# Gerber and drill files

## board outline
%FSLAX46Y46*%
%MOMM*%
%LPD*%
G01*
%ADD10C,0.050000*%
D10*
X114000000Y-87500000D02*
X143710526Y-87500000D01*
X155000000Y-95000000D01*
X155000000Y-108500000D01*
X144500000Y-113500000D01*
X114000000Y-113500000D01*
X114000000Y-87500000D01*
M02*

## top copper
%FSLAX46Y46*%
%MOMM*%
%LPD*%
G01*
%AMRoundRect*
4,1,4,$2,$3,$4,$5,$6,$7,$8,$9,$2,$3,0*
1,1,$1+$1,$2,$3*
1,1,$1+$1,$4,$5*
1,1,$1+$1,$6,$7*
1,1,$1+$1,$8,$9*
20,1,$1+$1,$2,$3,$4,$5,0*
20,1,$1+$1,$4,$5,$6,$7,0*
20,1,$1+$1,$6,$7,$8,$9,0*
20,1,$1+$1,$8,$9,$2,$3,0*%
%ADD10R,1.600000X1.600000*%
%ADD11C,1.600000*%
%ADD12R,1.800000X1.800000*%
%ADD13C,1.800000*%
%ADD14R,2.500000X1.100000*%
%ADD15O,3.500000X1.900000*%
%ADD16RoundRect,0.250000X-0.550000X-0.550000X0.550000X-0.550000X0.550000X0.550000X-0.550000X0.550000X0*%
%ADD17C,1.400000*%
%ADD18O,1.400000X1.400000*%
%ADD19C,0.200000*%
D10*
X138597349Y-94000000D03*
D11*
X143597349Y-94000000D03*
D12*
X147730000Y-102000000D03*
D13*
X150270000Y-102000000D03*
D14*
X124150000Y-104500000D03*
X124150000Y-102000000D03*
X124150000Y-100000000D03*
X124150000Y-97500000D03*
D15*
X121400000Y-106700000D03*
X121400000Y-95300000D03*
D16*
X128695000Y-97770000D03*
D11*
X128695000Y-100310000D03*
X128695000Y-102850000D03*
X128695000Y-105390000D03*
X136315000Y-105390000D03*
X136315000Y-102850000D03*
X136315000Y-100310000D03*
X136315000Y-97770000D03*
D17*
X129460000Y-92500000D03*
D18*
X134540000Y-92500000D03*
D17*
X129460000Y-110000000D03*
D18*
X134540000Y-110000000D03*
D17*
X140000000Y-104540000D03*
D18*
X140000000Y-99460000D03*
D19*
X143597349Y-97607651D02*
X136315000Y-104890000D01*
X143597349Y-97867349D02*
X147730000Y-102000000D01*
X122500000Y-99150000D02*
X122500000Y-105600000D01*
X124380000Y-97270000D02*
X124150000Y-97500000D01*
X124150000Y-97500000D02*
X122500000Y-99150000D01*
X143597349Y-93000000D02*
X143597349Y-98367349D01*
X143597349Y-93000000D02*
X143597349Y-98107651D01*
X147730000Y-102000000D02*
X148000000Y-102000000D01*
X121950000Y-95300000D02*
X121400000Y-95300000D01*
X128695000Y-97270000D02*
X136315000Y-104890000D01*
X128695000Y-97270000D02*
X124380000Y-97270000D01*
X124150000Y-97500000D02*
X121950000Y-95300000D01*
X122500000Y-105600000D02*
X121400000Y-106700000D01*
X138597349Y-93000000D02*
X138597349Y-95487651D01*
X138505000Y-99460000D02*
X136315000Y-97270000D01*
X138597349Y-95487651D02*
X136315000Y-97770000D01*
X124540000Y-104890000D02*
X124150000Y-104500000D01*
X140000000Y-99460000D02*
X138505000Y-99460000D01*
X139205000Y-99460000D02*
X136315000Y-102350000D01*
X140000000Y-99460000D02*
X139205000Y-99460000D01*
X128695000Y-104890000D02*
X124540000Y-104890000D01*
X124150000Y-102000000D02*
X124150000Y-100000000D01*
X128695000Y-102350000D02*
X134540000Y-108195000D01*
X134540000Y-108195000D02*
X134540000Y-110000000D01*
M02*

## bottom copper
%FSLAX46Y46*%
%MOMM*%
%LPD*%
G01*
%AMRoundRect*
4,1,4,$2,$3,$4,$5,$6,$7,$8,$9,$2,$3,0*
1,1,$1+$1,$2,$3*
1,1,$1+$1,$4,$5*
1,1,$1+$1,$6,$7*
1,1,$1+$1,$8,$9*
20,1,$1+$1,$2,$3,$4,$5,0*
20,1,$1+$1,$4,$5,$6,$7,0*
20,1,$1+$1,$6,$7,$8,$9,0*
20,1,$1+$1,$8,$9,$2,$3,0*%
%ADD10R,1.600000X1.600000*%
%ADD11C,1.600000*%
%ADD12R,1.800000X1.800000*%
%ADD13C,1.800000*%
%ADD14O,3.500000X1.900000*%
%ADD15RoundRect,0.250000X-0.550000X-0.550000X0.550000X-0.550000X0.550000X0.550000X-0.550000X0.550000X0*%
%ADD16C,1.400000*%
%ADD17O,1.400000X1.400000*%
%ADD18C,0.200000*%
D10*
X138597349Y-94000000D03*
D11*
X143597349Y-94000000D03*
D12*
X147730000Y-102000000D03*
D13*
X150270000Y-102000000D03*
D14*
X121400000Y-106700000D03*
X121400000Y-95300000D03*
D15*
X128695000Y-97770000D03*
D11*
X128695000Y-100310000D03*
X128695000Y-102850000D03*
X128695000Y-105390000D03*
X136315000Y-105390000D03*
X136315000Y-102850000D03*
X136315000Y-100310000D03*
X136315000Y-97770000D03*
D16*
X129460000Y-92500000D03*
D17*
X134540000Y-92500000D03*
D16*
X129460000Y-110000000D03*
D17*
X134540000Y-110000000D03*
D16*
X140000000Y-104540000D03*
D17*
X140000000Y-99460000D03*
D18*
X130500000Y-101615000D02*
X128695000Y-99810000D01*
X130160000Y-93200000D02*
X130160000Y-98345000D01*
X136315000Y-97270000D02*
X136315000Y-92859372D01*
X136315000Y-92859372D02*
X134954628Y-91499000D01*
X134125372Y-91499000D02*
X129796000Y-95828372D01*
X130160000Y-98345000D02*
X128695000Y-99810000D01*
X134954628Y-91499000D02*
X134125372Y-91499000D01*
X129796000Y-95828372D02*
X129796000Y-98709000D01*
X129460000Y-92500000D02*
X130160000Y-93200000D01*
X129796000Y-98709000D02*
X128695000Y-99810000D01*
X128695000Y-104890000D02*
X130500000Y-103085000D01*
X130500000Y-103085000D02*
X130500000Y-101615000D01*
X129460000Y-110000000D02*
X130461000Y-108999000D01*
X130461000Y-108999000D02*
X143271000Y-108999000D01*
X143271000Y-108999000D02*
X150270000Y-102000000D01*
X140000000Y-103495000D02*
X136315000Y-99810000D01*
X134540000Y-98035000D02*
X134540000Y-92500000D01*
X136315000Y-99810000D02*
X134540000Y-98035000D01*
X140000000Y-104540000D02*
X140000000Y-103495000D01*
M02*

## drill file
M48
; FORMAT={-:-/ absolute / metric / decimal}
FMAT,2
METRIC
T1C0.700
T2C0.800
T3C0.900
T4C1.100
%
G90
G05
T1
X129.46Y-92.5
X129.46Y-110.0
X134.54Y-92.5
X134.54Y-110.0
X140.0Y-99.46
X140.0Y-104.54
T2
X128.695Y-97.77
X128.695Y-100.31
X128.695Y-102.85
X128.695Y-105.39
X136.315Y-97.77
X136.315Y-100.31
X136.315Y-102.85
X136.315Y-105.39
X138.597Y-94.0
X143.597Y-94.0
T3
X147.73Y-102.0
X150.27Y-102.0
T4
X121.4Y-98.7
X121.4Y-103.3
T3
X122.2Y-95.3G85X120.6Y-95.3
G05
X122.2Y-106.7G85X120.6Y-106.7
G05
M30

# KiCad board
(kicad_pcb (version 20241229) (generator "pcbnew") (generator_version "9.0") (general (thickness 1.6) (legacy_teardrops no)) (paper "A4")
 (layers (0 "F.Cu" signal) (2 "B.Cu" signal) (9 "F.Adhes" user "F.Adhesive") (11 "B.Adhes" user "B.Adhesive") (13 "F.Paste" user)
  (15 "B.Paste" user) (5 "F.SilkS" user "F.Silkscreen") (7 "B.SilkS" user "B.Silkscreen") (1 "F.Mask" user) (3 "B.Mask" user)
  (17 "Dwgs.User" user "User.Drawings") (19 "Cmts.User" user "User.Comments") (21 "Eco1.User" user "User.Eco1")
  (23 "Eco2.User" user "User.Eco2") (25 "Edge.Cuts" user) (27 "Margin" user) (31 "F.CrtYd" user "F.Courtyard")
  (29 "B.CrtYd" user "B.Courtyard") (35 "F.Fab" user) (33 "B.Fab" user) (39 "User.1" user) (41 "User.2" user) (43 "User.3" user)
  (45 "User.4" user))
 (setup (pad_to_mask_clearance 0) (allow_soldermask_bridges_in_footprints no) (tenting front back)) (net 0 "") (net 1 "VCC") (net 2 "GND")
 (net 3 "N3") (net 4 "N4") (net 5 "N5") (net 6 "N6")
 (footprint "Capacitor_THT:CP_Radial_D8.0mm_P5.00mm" (layer "F.Cu") (at 138.597349 94)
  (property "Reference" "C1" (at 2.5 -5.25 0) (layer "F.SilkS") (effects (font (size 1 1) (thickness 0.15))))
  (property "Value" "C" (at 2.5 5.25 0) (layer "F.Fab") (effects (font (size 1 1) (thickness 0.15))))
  (pad "1" thru_hole rect (at 0 0) (size 1.6 1.6) (drill 0.8) (layers "*.Cu" "*.Mask") (remove_unused_layers no) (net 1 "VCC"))
  (pad "2" thru_hole circle (at 5 0) (size 1.6 1.6) (drill 0.8) (layers "*.Cu" "*.Mask") (remove_unused_layers no) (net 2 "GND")))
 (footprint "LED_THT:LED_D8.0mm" (layer "F.Cu") (at 147.73 102)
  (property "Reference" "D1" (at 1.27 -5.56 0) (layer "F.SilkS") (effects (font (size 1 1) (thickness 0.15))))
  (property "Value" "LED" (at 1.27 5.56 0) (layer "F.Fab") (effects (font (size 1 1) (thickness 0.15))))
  (pad "1" thru_hole rect (at 0 0) (size 1.8 1.8) (drill 0.9) (layers "*.Cu" "*.Mask") (remove_unused_layers no) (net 2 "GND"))
  (pad "2" thru_hole circle (at 2.54 0) (size 1.8 1.8) (drill 0.9) (layers "*.Cu" "*.Mask") (remove_unused_layers no) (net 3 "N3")))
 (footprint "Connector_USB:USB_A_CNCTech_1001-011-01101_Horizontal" (layer "F.Cu") (at 114.5 101 180)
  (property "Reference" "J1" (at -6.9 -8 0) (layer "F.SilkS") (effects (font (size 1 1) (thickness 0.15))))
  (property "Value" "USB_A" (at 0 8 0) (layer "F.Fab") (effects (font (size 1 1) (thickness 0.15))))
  (pad "" np_thru_hole circle (at -6.9 -2.3 180) (size 1.1 1.1) (drill 1.1) (layers "*.Cu" "*.Mask"))
  (pad "" np_thru_hole circle (at -6.9 2.3 180) (size 1.1 1.1) (drill 1.1) (layers "*.Cu" "*.Mask"))
  (pad "1" smd rect (at -9.65 -3.5 180) (size 2.5 1.1) (layers "F.Cu" "F.Mask" "F.Paste") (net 1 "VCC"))
  (pad "2" smd rect (at -9.65 -1 180) (size 2.5 1.1) (layers "F.Cu" "F.Mask" "F.Paste") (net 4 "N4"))
  (pad "3" smd rect (at -9.65 1 180) (size 2.5 1.1) (layers "F.Cu" "F.Mask" "F.Paste") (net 4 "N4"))
  (pad "4" smd rect (at -9.65 3.5 180) (size 2.5 1.1) (layers "F.Cu" "F.Mask" "F.Paste") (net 2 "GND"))
  (pad "5" thru_hole oval (at -6.9 -5.7 180) (size 3.5 1.9) (drill oval 2.5 0.9) (layers "*.Cu" "*.Mask") (remove_unused_layers no)
   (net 2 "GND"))
  (pad "5" thru_hole oval (at -6.9 5.7 180) (size 3.5 1.9) (drill oval 2.5 0.9) (layers "*.Cu" "*.Mask") (remove_unused_layers no)
   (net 2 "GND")))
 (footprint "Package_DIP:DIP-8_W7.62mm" (layer "F.Cu") (at 128.695 97.77)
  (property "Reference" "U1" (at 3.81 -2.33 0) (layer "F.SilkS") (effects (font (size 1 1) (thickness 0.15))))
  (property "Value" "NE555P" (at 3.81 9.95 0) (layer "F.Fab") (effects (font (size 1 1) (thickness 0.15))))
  (pad "1" thru_hole roundrect (at 0 0) (size 1.6 1.6) (drill 0.8) (layers "*.Cu" "*.Mask") (remove_unused_layers no)
   (roundrect_rratio 0.15625) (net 2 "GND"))
  (pad "2" thru_hole circle (at 0 2.54) (size 1.6 1.6) (drill 0.8) (layers "*.Cu" "*.Mask") (remove_unused_layers no) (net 1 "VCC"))
  (pad "3" thru_hole circle (at 0 5.08) (size 1.6 1.6) (drill 0.8) (layers "*.Cu" "*.Mask") (remove_unused_layers no) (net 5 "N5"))
  (pad "4" thru_hole circle (at 0 7.62) (size 1.6 1.6) (drill 0.8) (layers "*.Cu" "*.Mask") (remove_unused_layers no) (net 1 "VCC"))
  (pad "5" thru_hole circle (at 7.62 7.62) (size 1.6 1.6) (drill 0.8) (layers "*.Cu" "*.Mask") (remove_unused_layers no) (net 2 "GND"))
  (pad "6" thru_hole circle (at 7.62 5.08) (size 1.6 1.6) (drill 0.8) (layers "*.Cu" "*.Mask") (remove_unused_layers no) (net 1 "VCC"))
  (pad "7" thru_hole circle (at 7.62 2.54) (size 1.6 1.6) (drill 0.8) (layers "*.Cu" "*.Mask") (remove_unused_layers no) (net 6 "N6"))
  (pad "8" thru_hole circle (at 7.62 0) (size 1.6 1.6) (drill 0.8) (layers "*.Cu" "*.Mask") (remove_unused_layers no) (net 1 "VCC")))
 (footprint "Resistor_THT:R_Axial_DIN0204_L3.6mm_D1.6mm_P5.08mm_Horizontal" (layer "F.Cu") (at 129.46 92.5)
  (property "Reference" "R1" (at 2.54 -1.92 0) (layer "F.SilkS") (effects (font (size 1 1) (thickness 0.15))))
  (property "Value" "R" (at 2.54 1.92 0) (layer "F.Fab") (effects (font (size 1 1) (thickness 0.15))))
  (pad "1" thru_hole circle (at 0 0) (size 1.4 1.4) (drill 0.7) (layers "*.Cu" "*.Mask") (remove_unused_layers no) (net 1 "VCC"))
  (pad "2" thru_hole oval (at 5.08 0) (size 1.4 1.4) (drill 0.7) (layers "*.Cu" "*.Mask") (remove_unused_layers no) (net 6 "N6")))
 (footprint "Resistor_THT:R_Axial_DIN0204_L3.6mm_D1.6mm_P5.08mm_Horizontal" (layer "F.Cu") (at 129.46 110)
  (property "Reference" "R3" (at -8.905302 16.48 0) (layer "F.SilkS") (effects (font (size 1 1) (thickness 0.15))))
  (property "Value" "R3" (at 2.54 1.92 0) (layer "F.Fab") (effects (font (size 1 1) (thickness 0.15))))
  (pad "1" thru_hole circle (at 0 0) (size 1.4 1.4) (drill 0.7) (layers "*.Cu" "*.Mask") (remove_unused_layers no) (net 3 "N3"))
  (pad "2" thru_hole oval (at 5.08 0) (size 1.4 1.4) (drill 0.7) (layers "*.Cu" "*.Mask") (remove_unused_layers no) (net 5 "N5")))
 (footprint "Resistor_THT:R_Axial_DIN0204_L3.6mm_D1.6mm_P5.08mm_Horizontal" (layer "F.Cu") (at 140 104.54 90)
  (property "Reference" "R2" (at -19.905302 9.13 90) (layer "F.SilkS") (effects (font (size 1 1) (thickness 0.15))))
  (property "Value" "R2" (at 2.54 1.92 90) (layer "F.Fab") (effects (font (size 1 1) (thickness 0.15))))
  (pad "1" thru_hole circle (at 0 0 90) (size 1.4 1.4) (drill 0.7) (layers "*.Cu" "*.Mask") (remove_unused_layers no) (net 6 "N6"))
  (pad "2" thru_hole oval (at 5.08 0 90) (size 1.4 1.4) (drill 0.7) (layers "*.Cu" "*.Mask") (remove_unused_layers no) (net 1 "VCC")))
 (gr_poly
  (pts (xy 114 87.5) (xy 143.710526 87.5) (xy 155 95) (xy 155 108.5) (xy 144.5 113.5) (xy 114 113.5)) (stroke (width 0.05) (type solid))
  (fill no) (layer "Edge.Cuts"))
 (segment (start 143.597349 97.607651) (end 136.315 104.89) (width 0.2) (layer "F.Cu") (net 2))
 (segment (start 143.597349 97.867349) (end 147.73 102) (width 0.2) (layer "F.Cu") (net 2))
 (segment (start 122.5 99.15) (end 122.5 105.6) (width 0.2) (layer "F.Cu") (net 2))
 (segment (start 124.38 97.27) (end 124.15 97.5) (width 0.2) (layer "F.Cu") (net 2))
 (segment (start 124.15 97.5) (end 122.5 99.15) (width 0.2) (layer "F.Cu") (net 2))
 (segment (start 143.597349 93) (end 143.597349 98.367349) (width 0.2) (layer "F.Cu") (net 2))
 (segment (start 143.597349 93) (end 143.597349 98.107651) (width 0.2) (layer "F.Cu") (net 2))
 (segment (start 147.73 102) (end 148 102) (width 0.2) (layer "F.Cu") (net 2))
 (segment (start 121.95 95.3) (end 121.4 95.3) (width 0.2) (layer "F.Cu") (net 2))
 (segment (start 128.695 97.27) (end 136.315 104.89) (width 0.2) (layer "F.Cu") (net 2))
 (segment (start 128.695 97.27) (end 124.38 97.27) (width 0.2) (layer "F.Cu") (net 2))
 (segment (start 124.15 97.5) (end 121.95 95.3) (width 0.2) (layer "F.Cu") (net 2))
 (segment (start 122.5 105.6) (end 121.4 106.7) (width 0.2) (layer "F.Cu") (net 2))
 (segment (start 138.597349 93) (end 138.597349 95.487651) (width 0.2) (layer "F.Cu") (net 1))
 (segment (start 138.505 99.46) (end 136.315 97.27) (width 0.2) (layer "F.Cu") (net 1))
 (segment (start 138.597349 95.487651) (end 136.315 97.77) (width 0.2) (layer "F.Cu") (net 1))
 (segment (start 124.54 104.89) (end 124.15 104.5) (width 0.2) (layer "F.Cu") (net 1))
 (segment (start 140 99.46) (end 138.505 99.46) (width 0.2) (layer "F.Cu") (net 1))
 (segment (start 139.205 99.46) (end 136.315 102.35) (width 0.2) (layer "F.Cu") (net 1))
 (segment (start 140 99.46) (end 139.205 99.46) (width 0.2) (layer "F.Cu") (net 1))
 (segment (start 128.695 104.89) (end 124.54 104.89) (width 0.2) (layer "F.Cu") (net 1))
 (segment (start 130.5 101.615) (end 128.695 99.81) (width 0.2) (layer "B.Cu") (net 1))
 (segment (start 130.16 93.2) (end 130.16 98.345) (width 0.2) (layer "B.Cu") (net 1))
 (segment (start 136.315 97.27) (end 136.315 92.859372) (width 0.2) (layer "B.Cu") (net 1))
 (segment (start 136.315 92.859372) (end 134.954628 91.499) (width 0.2) (layer "B.Cu") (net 1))
 (segment (start 134.125372 91.499) (end 129.796 95.828372) (width 0.2) (layer "B.Cu") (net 1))
 (segment (start 130.16 98.345) (end 128.695 99.81) (width 0.2) (layer "B.Cu") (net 1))
 (segment (start 134.954628 91.499) (end 134.125372 91.499) (width 0.2) (layer "B.Cu") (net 1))
 (segment (start 129.796 95.828372) (end 129.796 98.709) (width 0.2) (layer "B.Cu") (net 1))
 (segment (start 129.46 92.5) (end 130.16 93.2) (width 0.2) (layer "B.Cu") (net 1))
 (segment (start 129.796 98.709) (end 128.695 99.81) (width 0.2) (layer "B.Cu") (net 1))
 (segment (start 128.695 104.89) (end 130.5 103.085) (width 0.2) (layer "B.Cu") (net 1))
 (segment (start 130.5 103.085) (end 130.5 101.615) (width 0.2) (layer "B.Cu") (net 1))
 (segment (start 129.46 110) (end 130.461 108.999) (width 0.2) (layer "B.Cu") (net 3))
 (segment (start 130.461 108.999) (end 143.271 108.999) (width 0.2) (layer "B.Cu") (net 3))
 (segment (start 143.271 108.999) (end 150.27 102) (width 0.2) (layer "B.Cu") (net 3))
 (segment (start 124.15 102) (end 124.15 100) (width 0.2) (layer "F.Cu") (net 4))
 (segment (start 140 103.495) (end 136.315 99.81) (width 0.2) (layer "B.Cu") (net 6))
 (segment (start 134.54 98.035) (end 134.54 92.5) (width 0.2) (layer "B.Cu") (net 6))
 (segment (start 136.315 99.81) (end 134.54 98.035) (width 0.2) (layer "B.Cu") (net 6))
 (segment (start 140 104.54) (end 140 103.495) (width 0.2) (layer "B.Cu") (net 6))
 (segment (start 128.695 102.35) (end 134.54 108.195) (width 0.2) (layer "F.Cu") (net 5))
 (segment (start 134.54 108.195) (end 134.54 110) (width 0.2) (layer "F.Cu") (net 5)))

